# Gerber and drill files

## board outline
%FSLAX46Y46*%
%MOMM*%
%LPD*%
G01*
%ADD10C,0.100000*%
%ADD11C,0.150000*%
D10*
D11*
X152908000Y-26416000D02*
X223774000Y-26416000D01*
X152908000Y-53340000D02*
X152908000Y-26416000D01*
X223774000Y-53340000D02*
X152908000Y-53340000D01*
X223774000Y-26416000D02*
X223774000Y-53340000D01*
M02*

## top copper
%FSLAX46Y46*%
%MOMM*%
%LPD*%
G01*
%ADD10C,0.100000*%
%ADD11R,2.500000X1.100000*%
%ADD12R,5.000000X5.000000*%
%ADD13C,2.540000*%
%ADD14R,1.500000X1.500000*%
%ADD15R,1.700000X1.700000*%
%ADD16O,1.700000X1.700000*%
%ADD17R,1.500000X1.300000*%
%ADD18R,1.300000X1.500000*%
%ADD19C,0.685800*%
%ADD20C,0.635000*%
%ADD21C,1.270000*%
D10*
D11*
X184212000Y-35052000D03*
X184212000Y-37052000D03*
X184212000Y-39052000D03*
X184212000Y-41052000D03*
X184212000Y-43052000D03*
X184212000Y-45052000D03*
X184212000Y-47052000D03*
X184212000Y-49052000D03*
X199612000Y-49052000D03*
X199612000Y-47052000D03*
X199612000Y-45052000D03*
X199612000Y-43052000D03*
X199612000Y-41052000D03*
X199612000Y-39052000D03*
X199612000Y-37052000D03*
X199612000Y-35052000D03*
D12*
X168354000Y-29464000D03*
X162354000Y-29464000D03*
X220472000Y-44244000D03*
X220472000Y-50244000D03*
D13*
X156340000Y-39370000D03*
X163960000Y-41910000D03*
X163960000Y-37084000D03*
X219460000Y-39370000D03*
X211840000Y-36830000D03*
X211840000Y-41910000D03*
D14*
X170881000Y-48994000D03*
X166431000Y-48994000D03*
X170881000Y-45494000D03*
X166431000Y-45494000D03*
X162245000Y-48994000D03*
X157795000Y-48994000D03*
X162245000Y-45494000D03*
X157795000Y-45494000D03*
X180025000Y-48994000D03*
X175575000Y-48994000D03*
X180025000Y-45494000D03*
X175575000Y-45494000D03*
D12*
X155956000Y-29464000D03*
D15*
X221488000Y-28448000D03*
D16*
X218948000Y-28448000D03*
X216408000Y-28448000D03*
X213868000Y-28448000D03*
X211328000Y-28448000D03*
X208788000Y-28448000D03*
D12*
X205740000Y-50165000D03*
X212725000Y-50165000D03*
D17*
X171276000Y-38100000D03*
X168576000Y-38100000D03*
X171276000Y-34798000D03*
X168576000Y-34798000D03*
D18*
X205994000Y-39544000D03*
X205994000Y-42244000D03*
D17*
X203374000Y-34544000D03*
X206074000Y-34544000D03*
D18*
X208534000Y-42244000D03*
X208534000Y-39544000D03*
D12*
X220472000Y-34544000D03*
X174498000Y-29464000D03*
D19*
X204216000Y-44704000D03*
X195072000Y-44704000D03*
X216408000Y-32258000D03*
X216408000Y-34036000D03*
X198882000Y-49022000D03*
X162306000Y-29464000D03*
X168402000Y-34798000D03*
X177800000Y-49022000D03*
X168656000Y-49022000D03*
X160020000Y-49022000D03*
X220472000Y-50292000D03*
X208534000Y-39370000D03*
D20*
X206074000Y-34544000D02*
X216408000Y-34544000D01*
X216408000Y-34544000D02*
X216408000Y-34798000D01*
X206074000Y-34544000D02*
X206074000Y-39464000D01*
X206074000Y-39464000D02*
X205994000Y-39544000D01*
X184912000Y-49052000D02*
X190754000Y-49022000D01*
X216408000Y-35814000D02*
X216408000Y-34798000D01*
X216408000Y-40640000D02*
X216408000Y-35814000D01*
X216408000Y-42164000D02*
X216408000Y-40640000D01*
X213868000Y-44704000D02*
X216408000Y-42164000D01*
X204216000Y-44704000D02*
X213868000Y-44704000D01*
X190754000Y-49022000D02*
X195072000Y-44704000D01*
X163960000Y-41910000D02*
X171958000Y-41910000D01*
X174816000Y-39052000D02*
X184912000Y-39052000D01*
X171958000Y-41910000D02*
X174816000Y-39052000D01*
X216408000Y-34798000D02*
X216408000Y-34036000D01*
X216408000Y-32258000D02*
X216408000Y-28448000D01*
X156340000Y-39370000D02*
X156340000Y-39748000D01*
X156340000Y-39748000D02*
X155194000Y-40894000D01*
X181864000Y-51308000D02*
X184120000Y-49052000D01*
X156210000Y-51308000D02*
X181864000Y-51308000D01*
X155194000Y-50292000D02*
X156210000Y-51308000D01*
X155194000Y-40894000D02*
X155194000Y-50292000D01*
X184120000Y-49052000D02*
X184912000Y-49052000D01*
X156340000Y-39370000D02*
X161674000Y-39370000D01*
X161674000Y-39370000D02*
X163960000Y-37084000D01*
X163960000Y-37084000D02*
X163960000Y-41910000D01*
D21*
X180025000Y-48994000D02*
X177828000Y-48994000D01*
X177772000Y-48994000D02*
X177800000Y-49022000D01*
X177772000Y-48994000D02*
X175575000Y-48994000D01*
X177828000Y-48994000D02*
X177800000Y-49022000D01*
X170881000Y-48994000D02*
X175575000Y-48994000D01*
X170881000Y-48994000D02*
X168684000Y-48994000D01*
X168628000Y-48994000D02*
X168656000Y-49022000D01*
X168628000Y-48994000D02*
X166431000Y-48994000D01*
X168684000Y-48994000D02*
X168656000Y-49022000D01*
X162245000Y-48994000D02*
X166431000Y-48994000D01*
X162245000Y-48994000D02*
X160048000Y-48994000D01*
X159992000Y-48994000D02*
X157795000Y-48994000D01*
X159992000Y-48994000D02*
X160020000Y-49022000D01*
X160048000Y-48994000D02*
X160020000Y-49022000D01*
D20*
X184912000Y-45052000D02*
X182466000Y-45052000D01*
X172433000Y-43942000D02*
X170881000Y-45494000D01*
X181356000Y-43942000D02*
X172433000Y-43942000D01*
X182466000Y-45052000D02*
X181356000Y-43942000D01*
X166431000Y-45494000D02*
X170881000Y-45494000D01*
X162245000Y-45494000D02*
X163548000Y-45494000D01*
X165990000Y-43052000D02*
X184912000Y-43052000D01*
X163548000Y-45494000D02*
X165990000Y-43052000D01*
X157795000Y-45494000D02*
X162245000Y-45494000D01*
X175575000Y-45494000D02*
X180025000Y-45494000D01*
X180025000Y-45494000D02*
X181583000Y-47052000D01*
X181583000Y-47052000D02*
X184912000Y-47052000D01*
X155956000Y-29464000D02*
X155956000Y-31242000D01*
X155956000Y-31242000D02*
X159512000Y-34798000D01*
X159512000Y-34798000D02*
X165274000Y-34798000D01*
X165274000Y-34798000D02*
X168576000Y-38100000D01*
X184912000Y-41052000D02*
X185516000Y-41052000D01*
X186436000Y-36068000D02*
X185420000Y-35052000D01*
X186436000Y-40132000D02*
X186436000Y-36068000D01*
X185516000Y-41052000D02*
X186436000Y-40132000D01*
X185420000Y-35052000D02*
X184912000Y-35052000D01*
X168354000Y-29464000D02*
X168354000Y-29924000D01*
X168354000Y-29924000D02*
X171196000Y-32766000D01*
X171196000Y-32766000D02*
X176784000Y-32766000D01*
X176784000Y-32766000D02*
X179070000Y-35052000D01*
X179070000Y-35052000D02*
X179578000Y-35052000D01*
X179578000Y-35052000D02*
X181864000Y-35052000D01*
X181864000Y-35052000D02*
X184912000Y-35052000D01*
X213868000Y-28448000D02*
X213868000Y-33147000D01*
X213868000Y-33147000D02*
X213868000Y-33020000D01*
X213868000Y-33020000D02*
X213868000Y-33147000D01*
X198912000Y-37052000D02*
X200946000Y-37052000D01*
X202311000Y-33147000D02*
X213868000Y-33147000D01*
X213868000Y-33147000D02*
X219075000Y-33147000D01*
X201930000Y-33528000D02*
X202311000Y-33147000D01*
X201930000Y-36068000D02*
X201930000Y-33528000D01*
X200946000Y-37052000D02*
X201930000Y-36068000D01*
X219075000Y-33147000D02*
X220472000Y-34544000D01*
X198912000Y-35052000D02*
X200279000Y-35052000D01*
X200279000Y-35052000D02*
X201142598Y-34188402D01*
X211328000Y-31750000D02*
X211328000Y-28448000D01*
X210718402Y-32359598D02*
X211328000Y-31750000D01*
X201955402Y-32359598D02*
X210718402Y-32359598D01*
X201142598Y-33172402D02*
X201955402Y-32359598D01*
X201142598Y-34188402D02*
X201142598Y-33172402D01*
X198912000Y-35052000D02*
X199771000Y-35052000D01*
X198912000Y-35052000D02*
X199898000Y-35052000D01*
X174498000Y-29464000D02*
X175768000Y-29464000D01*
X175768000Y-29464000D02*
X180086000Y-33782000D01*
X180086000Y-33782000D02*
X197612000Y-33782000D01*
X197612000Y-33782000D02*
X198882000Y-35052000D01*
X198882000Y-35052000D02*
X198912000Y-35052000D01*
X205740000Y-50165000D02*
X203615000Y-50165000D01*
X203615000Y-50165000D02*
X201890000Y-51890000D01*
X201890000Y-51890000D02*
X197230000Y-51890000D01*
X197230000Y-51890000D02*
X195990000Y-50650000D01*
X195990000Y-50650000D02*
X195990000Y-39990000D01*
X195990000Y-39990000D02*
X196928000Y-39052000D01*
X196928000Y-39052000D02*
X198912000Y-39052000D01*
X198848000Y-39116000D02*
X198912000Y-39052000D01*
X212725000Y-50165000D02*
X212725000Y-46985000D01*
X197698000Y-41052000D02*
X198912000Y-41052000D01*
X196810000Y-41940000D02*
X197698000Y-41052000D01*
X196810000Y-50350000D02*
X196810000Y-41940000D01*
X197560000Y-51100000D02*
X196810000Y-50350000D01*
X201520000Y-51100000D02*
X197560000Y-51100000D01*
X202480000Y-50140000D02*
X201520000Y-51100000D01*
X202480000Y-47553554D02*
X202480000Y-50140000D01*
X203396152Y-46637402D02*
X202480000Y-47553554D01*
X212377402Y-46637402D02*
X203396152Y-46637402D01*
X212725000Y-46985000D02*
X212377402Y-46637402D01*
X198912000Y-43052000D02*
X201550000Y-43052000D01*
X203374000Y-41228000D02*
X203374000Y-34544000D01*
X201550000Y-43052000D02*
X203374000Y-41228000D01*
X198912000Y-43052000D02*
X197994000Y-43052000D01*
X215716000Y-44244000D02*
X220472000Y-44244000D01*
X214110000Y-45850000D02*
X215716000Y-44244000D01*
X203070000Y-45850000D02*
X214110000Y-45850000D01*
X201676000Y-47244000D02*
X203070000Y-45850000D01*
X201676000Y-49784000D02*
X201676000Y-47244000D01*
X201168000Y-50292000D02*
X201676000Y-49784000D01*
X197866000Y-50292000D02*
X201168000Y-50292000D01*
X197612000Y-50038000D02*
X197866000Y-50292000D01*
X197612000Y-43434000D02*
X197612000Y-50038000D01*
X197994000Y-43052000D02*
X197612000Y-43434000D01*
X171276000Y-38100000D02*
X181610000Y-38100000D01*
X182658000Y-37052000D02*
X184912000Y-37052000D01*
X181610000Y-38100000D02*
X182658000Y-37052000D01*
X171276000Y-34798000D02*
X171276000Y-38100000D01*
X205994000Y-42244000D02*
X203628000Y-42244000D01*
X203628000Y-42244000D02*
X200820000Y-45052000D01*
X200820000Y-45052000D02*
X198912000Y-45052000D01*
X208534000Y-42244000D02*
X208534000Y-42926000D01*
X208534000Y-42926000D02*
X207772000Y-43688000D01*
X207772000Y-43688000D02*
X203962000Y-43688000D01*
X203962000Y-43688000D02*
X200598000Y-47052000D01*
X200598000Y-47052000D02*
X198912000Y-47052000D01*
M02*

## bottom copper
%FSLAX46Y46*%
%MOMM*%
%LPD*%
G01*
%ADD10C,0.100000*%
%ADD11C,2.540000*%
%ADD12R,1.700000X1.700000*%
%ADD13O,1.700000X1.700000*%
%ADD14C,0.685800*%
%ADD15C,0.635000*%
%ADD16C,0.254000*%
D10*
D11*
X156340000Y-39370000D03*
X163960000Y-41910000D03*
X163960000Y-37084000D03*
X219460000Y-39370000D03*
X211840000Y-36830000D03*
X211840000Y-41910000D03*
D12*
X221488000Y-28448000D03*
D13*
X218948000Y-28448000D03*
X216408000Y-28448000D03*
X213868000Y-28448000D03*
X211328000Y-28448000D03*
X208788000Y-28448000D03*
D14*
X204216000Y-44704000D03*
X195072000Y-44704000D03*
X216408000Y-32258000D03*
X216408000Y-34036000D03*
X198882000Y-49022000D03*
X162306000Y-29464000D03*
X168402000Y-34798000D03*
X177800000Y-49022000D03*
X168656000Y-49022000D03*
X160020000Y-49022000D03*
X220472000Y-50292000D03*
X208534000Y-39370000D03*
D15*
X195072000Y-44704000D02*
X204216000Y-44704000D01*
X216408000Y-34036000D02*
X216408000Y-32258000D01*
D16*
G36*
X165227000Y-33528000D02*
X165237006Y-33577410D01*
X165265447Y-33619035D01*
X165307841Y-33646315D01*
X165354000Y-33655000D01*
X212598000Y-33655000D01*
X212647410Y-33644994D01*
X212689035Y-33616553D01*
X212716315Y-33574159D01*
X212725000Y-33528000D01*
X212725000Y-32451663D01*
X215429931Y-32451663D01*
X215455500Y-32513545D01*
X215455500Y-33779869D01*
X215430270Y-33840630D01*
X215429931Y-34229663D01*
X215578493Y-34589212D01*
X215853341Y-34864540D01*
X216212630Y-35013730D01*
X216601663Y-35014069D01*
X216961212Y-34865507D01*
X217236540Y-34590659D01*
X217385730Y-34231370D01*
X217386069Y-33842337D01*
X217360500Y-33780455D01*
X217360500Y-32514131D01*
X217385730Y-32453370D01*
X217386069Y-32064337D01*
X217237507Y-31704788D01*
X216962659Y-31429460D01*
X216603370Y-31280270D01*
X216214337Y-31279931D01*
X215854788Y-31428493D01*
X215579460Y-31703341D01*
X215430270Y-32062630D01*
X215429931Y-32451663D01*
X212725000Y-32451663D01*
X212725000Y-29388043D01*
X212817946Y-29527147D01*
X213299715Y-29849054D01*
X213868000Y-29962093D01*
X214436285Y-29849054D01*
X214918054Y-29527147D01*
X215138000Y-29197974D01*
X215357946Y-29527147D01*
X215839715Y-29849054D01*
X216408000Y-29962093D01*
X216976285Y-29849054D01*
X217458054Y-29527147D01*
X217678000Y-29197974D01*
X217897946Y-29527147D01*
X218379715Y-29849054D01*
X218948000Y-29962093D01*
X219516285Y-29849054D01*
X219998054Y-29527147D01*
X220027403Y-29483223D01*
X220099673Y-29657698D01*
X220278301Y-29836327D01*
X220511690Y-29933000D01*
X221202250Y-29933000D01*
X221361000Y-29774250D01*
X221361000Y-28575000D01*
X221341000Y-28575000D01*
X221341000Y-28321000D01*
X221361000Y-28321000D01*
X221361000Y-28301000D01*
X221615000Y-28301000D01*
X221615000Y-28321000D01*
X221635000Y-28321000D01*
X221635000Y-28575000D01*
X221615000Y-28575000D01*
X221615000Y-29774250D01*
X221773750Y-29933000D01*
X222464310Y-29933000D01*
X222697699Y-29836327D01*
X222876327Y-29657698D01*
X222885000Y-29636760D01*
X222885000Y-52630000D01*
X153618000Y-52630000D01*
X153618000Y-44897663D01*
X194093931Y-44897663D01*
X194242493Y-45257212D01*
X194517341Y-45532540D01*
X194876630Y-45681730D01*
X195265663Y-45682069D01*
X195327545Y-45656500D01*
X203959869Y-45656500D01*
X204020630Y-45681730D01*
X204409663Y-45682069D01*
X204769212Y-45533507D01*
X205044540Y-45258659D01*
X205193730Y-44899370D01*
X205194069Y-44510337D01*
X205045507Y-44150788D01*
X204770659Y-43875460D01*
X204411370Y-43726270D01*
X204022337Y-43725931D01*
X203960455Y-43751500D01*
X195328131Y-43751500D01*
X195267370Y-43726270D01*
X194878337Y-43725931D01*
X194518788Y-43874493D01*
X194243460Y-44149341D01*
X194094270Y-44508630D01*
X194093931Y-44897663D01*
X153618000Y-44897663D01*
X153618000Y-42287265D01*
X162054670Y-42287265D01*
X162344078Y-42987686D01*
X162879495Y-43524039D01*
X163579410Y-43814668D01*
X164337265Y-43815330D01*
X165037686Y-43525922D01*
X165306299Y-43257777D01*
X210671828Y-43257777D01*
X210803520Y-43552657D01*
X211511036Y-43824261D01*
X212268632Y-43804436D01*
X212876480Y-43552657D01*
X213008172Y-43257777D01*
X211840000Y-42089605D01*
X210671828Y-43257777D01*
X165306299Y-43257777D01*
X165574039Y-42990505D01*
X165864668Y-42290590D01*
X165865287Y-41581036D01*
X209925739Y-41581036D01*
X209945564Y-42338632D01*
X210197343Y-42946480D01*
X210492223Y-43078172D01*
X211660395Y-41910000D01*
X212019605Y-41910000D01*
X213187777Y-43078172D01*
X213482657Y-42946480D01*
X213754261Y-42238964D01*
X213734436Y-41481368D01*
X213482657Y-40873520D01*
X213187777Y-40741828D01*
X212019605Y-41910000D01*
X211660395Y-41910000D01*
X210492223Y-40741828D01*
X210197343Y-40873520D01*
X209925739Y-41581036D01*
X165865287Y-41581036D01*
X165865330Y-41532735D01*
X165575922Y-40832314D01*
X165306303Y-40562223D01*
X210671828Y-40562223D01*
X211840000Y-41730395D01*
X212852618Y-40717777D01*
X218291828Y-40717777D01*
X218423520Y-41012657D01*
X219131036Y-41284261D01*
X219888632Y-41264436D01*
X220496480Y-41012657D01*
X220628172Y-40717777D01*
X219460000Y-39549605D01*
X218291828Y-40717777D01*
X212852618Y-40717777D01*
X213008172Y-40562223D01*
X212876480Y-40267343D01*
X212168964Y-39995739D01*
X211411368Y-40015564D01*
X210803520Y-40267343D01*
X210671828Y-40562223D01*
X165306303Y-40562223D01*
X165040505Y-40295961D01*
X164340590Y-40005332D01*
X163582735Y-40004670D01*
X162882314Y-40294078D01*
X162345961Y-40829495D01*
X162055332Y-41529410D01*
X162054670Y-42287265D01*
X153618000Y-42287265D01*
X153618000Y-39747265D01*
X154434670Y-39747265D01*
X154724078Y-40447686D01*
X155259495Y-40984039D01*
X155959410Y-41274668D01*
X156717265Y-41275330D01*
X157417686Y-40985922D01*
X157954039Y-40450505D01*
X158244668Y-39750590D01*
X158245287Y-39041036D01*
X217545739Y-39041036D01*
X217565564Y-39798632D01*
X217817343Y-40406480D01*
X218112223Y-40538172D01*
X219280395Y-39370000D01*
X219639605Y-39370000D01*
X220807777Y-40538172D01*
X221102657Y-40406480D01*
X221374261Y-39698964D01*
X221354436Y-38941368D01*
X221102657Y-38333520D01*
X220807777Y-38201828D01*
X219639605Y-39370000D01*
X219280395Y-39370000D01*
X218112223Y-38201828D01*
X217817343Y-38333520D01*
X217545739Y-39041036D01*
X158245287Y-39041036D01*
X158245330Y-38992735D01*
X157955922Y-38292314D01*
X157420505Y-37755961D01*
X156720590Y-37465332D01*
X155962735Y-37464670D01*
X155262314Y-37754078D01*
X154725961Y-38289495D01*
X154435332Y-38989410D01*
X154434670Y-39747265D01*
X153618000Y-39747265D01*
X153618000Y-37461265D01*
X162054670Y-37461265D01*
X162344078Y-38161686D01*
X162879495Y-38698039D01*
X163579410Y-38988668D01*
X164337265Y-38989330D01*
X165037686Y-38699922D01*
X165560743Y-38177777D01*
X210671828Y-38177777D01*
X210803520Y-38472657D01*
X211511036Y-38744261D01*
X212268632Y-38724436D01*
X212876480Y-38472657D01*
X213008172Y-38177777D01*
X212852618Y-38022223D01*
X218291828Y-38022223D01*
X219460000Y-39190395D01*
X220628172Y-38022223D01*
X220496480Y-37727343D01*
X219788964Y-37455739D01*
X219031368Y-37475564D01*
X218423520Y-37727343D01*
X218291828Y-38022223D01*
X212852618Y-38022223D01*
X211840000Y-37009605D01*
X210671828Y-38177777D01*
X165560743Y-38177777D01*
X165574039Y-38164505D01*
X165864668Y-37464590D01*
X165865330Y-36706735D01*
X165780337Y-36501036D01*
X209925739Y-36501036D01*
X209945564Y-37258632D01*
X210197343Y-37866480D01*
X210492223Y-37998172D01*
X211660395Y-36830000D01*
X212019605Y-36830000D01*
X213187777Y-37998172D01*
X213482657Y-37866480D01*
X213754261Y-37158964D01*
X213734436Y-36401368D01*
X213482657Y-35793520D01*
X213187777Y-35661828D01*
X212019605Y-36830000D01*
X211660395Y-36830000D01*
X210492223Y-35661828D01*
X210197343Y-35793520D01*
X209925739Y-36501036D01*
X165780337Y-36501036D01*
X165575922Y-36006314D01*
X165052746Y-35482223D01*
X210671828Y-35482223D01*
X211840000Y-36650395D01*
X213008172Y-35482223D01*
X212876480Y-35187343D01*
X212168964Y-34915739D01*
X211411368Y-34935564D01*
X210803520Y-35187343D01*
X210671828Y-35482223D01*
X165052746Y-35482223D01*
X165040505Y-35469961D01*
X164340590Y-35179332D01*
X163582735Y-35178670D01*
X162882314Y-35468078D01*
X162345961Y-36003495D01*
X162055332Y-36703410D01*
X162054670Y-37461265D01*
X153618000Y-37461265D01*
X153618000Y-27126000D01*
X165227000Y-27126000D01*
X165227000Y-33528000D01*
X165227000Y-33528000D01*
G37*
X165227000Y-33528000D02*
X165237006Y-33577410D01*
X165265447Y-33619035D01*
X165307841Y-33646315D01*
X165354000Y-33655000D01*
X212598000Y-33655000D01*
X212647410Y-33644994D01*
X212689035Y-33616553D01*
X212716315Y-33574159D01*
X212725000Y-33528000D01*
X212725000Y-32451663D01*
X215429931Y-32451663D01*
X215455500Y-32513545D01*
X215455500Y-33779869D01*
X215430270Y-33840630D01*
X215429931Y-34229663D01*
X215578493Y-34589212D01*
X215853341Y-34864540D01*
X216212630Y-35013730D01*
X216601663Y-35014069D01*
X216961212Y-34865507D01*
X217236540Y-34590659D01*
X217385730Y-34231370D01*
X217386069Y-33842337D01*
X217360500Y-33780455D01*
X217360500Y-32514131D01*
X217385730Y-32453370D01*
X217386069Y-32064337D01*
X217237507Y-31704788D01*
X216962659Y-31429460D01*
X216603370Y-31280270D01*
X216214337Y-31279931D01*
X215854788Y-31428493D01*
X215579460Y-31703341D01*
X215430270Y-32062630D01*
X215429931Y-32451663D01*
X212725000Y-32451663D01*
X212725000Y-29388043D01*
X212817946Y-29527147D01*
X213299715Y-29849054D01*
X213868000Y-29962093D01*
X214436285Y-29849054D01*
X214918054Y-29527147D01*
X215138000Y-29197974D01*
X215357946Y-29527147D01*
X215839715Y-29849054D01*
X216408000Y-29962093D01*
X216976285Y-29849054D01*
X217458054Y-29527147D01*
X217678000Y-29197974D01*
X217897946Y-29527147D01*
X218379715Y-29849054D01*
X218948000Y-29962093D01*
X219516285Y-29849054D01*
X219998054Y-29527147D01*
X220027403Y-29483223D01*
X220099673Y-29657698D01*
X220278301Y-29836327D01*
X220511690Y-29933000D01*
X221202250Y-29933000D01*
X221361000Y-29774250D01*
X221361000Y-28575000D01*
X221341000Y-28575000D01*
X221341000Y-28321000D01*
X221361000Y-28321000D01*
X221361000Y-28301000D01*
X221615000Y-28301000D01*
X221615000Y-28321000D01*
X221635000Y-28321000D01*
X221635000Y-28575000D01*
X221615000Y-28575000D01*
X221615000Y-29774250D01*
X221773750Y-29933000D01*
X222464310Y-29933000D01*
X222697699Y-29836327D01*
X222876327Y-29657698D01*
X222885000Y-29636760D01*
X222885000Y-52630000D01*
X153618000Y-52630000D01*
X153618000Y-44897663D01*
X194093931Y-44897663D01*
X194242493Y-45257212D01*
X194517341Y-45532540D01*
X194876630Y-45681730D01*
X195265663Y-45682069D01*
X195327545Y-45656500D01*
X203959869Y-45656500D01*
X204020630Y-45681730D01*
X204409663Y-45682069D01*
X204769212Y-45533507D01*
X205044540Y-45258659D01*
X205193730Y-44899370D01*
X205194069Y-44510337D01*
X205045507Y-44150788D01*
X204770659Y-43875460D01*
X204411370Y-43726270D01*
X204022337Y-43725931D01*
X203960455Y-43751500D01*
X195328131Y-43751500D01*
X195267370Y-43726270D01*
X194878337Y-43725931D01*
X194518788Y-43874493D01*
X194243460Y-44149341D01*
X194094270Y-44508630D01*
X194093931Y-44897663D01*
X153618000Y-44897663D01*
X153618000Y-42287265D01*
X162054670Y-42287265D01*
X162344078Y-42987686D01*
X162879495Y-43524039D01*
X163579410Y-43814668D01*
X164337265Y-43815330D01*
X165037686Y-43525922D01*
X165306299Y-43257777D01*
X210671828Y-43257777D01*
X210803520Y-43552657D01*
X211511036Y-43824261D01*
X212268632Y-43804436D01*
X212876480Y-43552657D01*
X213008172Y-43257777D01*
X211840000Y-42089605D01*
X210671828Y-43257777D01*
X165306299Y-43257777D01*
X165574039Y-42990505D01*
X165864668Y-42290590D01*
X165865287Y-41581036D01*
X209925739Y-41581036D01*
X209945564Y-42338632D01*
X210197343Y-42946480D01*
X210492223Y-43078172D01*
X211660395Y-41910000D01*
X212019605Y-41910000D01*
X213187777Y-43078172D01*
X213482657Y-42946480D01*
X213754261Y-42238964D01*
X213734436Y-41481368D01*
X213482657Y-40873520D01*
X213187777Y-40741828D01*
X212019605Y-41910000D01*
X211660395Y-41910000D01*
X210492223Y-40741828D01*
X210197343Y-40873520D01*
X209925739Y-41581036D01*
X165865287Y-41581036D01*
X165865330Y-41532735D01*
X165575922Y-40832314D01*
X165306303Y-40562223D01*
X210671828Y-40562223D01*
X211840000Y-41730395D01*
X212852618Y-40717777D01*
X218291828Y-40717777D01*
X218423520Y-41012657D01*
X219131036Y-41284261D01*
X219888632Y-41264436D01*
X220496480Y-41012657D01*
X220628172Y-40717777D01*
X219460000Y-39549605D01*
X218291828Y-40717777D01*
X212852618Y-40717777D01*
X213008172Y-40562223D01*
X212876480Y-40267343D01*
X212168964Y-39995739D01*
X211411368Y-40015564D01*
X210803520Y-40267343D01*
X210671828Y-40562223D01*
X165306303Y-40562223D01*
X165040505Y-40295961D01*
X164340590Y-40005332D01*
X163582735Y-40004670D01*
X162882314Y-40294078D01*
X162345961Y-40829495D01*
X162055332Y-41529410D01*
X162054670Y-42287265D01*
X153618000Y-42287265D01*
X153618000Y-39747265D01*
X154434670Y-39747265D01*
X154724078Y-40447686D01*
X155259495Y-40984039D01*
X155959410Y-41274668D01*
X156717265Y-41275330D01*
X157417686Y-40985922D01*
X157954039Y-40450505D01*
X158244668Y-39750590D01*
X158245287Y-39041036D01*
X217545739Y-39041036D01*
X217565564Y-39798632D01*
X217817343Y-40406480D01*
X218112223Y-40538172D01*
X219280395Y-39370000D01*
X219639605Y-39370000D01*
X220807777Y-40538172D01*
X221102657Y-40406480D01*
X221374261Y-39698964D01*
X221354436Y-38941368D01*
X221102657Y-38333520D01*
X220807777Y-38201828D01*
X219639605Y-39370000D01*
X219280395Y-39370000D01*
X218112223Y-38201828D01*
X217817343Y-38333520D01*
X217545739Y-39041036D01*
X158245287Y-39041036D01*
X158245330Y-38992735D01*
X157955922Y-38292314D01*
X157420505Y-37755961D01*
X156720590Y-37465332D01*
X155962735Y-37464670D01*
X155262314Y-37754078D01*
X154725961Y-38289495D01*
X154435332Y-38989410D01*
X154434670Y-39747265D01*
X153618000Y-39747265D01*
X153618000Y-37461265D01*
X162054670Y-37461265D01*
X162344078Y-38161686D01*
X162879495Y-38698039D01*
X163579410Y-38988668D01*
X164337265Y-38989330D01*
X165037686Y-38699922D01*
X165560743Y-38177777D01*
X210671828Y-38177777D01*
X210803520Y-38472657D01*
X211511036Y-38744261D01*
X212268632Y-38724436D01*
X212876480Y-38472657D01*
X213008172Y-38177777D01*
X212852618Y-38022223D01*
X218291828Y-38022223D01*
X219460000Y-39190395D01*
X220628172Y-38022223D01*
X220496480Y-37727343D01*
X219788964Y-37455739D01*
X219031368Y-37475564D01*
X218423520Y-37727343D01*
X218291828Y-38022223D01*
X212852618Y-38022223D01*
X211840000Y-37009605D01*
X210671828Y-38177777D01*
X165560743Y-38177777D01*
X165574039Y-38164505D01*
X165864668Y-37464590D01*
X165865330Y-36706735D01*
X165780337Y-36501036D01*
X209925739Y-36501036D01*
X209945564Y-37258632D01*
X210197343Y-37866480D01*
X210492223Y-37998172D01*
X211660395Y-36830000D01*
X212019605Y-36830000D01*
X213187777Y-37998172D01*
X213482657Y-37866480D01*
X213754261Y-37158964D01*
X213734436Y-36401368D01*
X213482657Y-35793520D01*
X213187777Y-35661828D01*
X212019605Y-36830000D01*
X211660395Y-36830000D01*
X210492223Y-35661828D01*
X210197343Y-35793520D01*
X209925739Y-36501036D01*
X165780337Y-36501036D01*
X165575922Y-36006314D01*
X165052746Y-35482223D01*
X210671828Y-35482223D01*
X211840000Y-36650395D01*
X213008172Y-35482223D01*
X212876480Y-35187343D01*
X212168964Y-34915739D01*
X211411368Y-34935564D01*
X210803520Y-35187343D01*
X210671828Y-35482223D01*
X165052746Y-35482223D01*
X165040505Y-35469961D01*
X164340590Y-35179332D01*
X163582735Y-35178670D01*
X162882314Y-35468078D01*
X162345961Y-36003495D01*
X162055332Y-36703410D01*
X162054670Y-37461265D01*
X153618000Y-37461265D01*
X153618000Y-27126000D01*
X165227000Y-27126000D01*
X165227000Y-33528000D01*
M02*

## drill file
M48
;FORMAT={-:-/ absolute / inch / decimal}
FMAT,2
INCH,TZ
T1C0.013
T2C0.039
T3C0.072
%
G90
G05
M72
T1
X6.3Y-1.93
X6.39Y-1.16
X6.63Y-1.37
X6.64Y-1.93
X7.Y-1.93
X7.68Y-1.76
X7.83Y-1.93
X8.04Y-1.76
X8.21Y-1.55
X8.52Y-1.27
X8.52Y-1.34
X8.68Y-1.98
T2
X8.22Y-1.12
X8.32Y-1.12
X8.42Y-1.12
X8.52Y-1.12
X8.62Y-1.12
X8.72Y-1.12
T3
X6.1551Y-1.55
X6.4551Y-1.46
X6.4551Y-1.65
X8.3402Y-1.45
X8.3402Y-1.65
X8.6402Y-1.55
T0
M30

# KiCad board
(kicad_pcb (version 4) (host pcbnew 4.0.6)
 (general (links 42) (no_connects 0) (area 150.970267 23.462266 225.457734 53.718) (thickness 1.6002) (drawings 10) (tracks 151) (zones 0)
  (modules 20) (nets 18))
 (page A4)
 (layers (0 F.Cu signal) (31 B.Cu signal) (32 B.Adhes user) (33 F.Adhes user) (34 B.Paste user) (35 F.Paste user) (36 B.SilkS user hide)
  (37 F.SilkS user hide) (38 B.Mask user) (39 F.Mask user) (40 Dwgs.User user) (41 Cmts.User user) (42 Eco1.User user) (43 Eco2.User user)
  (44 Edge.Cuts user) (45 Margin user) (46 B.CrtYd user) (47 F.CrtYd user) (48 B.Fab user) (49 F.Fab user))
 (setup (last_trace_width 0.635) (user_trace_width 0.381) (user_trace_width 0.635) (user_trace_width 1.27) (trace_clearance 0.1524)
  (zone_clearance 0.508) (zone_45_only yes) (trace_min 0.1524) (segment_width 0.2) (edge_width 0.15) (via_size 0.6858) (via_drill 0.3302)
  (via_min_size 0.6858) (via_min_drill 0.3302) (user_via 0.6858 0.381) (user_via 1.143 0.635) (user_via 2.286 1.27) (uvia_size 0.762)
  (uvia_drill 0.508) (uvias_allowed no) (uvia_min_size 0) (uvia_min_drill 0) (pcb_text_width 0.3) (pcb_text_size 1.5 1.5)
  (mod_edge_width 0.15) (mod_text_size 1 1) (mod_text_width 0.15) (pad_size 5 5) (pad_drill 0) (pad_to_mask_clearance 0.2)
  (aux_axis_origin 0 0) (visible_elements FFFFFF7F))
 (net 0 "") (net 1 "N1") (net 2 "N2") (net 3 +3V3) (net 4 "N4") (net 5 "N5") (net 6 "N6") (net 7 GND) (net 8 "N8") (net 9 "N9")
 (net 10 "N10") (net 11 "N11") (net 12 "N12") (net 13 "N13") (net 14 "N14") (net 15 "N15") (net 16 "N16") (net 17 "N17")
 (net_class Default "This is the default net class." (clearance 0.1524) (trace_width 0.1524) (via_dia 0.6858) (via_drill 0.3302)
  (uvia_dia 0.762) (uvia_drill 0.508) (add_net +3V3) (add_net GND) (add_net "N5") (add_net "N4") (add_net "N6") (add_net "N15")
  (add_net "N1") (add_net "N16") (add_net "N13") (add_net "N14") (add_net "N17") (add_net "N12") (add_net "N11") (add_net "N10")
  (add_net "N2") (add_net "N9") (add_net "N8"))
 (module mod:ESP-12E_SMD (layer F.Cu) (at 184.912 35.052)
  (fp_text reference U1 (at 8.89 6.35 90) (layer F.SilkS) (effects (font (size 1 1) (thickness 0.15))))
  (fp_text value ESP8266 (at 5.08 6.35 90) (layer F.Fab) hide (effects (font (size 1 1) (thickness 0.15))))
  (pad 1 smd rect (at 0 0) (size 2.5 1.1) (drill (offset -0.7 0)) (layers F.Cu F.Paste F.Mask) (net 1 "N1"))
  (pad 2 smd rect (at 0 2) (size 2.5 1.1) (drill (offset -0.7 0)) (layers F.Cu F.Paste F.Mask) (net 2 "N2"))
  (pad 3 smd rect (at 0 4) (size 2.5 1.1) (drill (offset -0.7 0)) (layers F.Cu F.Paste F.Mask) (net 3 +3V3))
  (pad 4 smd rect (at 0 6) (size 2.5 1.1) (drill (offset -0.7 0)) (layers F.Cu F.Paste F.Mask) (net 1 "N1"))
  (pad 5 smd rect (at 0 8) (size 2.5 1.1) (drill (offset -0.7 0)) (layers F.Cu F.Paste F.Mask) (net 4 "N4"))
  (pad 6 smd rect (at 0 10) (size 2.5 1.1) (drill (offset -0.7 0)) (layers F.Cu F.Paste F.Mask) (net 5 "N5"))
  (pad 7 smd rect (at 0 12) (size 2.5 1.1) (drill (offset -0.7 0)) (layers F.Cu F.Paste F.Mask) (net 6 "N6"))
  (pad 8 smd rect (at 0 14) (size 2.5 1.1) (drill (offset -0.7 0)) (layers F.Cu F.Paste F.Mask) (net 3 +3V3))
  (pad 9 smd rect (at 14 14) (size 2.5 1.1) (drill (offset 0.7 0)) (layers F.Cu F.Paste F.Mask) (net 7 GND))
  (pad 10 smd rect (at 14 12) (size 2.5 1.1) (drill (offset 0.7 0)) (layers F.Cu F.Paste F.Mask) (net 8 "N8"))
  (pad 11 smd rect (at 14 10) (size 2.5 1.1) (drill (offset 0.7 0)) (layers F.Cu F.Paste F.Mask) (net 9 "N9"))
  (pad 12 smd rect (at 14 8) (size 2.5 1.1) (drill (offset 0.7 0)) (layers F.Cu F.Paste F.Mask) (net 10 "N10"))
  (pad 13 smd rect (at 14 6) (size 2.5 1.1) (drill (offset 0.7 0)) (layers F.Cu F.Paste F.Mask) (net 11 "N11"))
  (pad 14 smd rect (at 14 4) (size 2.5 1.1) (drill (offset 0.7 0)) (layers F.Cu F.Paste F.Mask) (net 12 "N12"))
  (pad 15 smd rect (at 14 2) (size 2.5 1.1) (drill (offset 0.7 0)) (layers F.Cu F.Paste F.Mask) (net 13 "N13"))
  (pad 16 smd rect (at 14 0) (size 2.5 1.1) (drill (offset 0.7 0)) (layers F.Cu F.Paste F.Mask) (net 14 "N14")))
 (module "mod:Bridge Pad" (layer F.Cu) (at 165.354 29.464)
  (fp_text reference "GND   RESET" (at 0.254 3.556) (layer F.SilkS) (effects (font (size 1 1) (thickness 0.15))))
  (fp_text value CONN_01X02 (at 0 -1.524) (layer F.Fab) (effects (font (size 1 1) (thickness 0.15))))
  (pad 1 smd rect (at 3 0) (size 5 5) (layers F.Cu F.Mask) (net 1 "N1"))
  (pad 2 smd rect (at -3 0) (size 5 5) (layers F.Cu F.Mask) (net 7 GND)))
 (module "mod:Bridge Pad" (layer F.Cu) (at 220.472 47.244 90)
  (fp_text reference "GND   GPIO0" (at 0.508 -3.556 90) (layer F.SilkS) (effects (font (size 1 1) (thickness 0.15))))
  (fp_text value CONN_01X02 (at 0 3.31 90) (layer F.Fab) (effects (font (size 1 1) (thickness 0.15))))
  (pad 1 smd rect (at 3 0 90) (size 5 5) (layers F.Cu F.Mask) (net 10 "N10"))
  (pad 2 smd rect (at -3 0 90) (size 5 5) (layers F.Cu F.Mask) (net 7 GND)))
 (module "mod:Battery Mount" (layer F.Cu) (at 187.96 39.37 90)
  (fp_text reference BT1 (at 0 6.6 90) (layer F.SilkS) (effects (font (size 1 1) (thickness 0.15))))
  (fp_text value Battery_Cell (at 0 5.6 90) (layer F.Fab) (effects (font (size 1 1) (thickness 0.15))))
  (pad 1 thru_hole circle (at 0 -31.62 90) (size 2.54 2.54) (drill 1.8288) (layers *.Cu *.Mask) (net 3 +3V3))
  (pad 1 thru_hole circle (at -2.54 -24 90) (size 2.54 2.54) (drill 1.8288) (layers *.Cu *.Mask) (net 3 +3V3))
  (pad 1 thru_hole circle (at 2.286 -24 90) (size 2.54 2.54) (drill 1.8288) (layers *.Cu *.Mask) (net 3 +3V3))
  (pad 2 thru_hole circle (at 0 31.5 90) (size 2.54 2.54) (drill 1.8288) (layers *.Cu *.Mask) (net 7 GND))
  (pad 2 thru_hole circle (at 2.54 23.88 90) (size 2.54 2.54) (drill 1.8288) (layers *.Cu *.Mask) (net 7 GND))
  (pad 2 thru_hole circle (at -2.54 23.88 90) (size 2.54 2.54) (drill 1.8288) (layers *.Cu *.Mask) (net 7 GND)))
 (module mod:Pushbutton (layer F.Cu) (at 168.656 47.244 180)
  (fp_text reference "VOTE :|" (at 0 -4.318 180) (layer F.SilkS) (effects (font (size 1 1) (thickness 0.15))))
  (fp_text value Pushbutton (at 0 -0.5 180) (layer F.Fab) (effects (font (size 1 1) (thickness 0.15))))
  (pad 1 smd rect (at -2.225 -1.75 180) (size 1.5 1.5) (layers F.Cu F.Paste F.Mask) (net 7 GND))
  (pad 1 smd rect (at 2.225 -1.75 180) (size 1.5 1.5) (layers F.Cu F.Paste F.Mask) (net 7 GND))
  (pad 2 smd rect (at -2.225 1.75 180) (size 1.5 1.5) (layers F.Cu F.Paste F.Mask) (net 5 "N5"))
  (pad 2 smd rect (at 2.225 1.75 180) (size 1.5 1.5) (layers F.Cu F.Paste F.Mask) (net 5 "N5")))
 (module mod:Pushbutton (layer F.Cu) (at 160.02 47.244 180)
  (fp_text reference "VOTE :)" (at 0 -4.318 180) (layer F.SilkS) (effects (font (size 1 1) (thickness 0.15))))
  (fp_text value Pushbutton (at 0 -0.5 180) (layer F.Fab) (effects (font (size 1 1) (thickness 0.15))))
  (pad 1 smd rect (at -2.225 -1.75 180) (size 1.5 1.5) (layers F.Cu F.Paste F.Mask) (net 7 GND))
  (pad 1 smd rect (at 2.225 -1.75 180) (size 1.5 1.5) (layers F.Cu F.Paste F.Mask) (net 7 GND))
  (pad 2 smd rect (at -2.225 1.75 180) (size 1.5 1.5) (layers F.Cu F.Paste F.Mask) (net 4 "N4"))
  (pad 2 smd rect (at 2.225 1.75 180) (size 1.5 1.5) (layers F.Cu F.Paste F.Mask) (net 4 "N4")))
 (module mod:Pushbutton (layer F.Cu) (at 177.8 47.244 180)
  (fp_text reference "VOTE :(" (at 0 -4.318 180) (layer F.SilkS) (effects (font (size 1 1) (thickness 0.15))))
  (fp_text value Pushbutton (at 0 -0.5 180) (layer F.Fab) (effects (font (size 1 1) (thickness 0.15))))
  (pad 1 smd rect (at -2.225 -1.75 180) (size 1.5 1.5) (layers F.Cu F.Paste F.Mask) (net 7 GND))
  (pad 1 smd rect (at 2.225 -1.75 180) (size 1.5 1.5) (layers F.Cu F.Paste F.Mask) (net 7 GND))
  (pad 2 smd rect (at -2.225 1.75 180) (size 1.5 1.5) (layers F.Cu F.Paste F.Mask) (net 6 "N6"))
  (pad 2 smd rect (at 2.225 1.75 180) (size 1.5 1.5) (layers F.Cu F.Paste F.Mask) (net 6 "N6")))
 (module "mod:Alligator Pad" (layer F.Cu) (at 155.956 29.464)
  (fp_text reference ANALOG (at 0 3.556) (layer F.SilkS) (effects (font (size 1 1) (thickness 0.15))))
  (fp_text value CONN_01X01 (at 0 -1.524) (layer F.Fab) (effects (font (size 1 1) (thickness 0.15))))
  (pad 1 smd rect (at 0 0) (size 5 5) (layers F.Cu F.Mask) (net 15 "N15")))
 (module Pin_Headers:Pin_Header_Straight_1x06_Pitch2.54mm (layer F.Cu) (at 221.488 28.448 270)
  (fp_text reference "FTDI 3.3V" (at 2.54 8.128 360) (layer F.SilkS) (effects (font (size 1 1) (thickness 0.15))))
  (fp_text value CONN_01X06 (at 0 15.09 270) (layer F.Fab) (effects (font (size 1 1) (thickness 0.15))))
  (pad 1 thru_hole rect (at 0 0 270) (size 1.7 1.7) (drill 1) (layers *.Cu *.Mask) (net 7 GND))
  (pad 2 thru_hole oval (at 0 2.54 270) (size 1.7 1.7) (drill 1) (layers *.Cu *.Mask) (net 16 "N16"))
  (pad 3 thru_hole oval (at 0 5.08 270) (size 1.7 1.7) (drill 1) (layers *.Cu *.Mask) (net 3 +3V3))
  (pad 4 thru_hole oval (at 0 7.62 270) (size 1.7 1.7) (drill 1) (layers *.Cu *.Mask) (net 13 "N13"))
  (pad 5 thru_hole oval (at 0 10.16 270) (size 1.7 1.7) (drill 1) (layers *.Cu *.Mask) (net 14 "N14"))
  (pad 6 thru_hole oval (at 0 12.7 270) (size 1.7 1.7) (drill 1) (layers *.Cu *.Mask) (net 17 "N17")))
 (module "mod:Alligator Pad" (layer F.Cu) (at 205.74 50.165)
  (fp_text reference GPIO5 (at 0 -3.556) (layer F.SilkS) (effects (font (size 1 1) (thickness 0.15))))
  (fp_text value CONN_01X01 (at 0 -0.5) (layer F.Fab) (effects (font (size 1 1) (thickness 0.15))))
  (pad 1 smd rect (at 0 0) (size 5 5) (layers F.Cu F.Mask) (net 12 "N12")))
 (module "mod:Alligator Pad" (layer F.Cu) (at 212.725 50.165)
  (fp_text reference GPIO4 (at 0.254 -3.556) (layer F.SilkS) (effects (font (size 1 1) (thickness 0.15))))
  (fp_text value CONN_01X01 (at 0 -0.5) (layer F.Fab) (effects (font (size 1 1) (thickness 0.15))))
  (pad 1 smd rect (at 0 0) (size 5 5) (layers F.Cu F.Mask) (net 11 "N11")))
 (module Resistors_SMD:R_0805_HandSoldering (layer F.Cu) (at 169.926 38.1 180)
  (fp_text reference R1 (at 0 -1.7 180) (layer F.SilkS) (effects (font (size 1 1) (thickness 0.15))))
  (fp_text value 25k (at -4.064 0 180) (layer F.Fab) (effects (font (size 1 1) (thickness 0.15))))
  (pad 1 smd rect (at -1.35 0 180) (size 1.5 1.3) (layers F.Cu F.Paste F.Mask) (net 2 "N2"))
  (pad 2 smd rect (at 1.35 0 180) (size 1.5 1.3) (layers F.Cu F.Paste F.Mask) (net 15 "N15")))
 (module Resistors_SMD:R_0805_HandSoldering (layer F.Cu) (at 169.926 34.798 180)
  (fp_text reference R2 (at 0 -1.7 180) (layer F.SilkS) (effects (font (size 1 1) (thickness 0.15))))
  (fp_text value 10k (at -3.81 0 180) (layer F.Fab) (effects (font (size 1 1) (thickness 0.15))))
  (pad 1 smd rect (at -1.35 0 180) (size 1.5 1.3) (layers F.Cu F.Paste F.Mask) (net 2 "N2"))
  (pad 2 smd rect (at 1.35 0 180) (size 1.5 1.3) (layers F.Cu F.Paste F.Mask) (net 7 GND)))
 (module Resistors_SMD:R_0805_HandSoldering (layer F.Cu) (at 205.994 40.894 270)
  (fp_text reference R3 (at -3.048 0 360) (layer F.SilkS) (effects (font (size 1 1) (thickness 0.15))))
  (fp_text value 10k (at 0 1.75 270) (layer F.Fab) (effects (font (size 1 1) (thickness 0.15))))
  (pad 1 smd rect (at -1.35 0 270) (size 1.5 1.3) (layers F.Cu F.Paste F.Mask) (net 3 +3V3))
  (pad 2 smd rect (at 1.35 0 270) (size 1.5 1.3) (layers F.Cu F.Paste F.Mask) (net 9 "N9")))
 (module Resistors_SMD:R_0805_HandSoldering (layer F.Cu) (at 204.724 34.544)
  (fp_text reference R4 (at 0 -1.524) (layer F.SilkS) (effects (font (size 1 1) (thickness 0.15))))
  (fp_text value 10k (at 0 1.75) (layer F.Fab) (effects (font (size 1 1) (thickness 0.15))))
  (pad 1 smd rect (at -1.35 0) (size 1.5 1.3) (layers F.Cu F.Paste F.Mask) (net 10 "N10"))
  (pad 2 smd rect (at 1.35 0) (size 1.5 1.3) (layers F.Cu F.Paste F.Mask) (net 3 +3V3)))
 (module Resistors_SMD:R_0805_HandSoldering (layer F.Cu) (at 208.534 40.894 90)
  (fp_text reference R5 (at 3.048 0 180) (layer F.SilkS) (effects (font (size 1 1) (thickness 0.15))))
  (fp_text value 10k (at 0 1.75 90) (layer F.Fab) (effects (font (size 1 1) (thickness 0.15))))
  (pad 1 smd rect (at -1.35 0 90) (size 1.5 1.3) (layers F.Cu F.Paste F.Mask) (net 8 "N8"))
  (pad 2 smd rect (at 1.35 0 90) (size 1.5 1.3) (layers F.Cu F.Paste F.Mask) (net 7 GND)))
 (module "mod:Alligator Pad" (layer F.Cu) (at 220.472 34.544)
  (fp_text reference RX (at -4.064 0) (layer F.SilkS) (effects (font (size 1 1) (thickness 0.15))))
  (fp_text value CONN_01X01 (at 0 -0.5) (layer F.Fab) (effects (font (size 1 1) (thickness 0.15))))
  (pad 1 smd rect (at 0 0) (size 5 5) (layers F.Cu F.Mask) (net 13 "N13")))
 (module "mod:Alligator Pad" (layer F.Cu) (at 174.498 29.464)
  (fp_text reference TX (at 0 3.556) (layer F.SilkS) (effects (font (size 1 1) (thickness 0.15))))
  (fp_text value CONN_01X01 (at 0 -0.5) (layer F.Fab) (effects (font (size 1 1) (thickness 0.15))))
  (pad 1 smd rect (at 0 0) (size 5 5) (layers F.Cu F.Mask) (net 14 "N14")))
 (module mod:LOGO (layer F.Cu) (at 177.292 38.1)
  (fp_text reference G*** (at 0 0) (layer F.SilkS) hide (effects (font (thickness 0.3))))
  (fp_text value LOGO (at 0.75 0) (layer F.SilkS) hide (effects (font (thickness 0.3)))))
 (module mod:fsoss (layer B.Cu) (at 159.258 47.244)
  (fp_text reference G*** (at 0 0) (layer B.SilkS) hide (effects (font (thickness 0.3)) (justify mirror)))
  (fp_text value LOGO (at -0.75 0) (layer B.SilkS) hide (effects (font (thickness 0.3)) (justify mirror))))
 (gr_line (start 152.908 26.416) (end 223.774 26.416) (angle 90) (layer Edge.Cuts) (width 0.15))
 (gr_line (start 152.908 53.34) (end 152.908 26.416) (angle 90) (layer Edge.Cuts) (width 0.15))
 (gr_line (start 223.774 53.34) (end 152.908 53.34) (angle 90) (layer Edge.Cuts) (width 0.15))
 (gr_line (start 223.774 26.416) (end 223.774 53.34) (angle 90) (layer Edge.Cuts) (width 0.15))
 (segment (start 206.074 34.544) (end 216.408 34.544) (width 0.635) (layer F.Cu) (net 3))
 (segment (start 216.408 34.544) (end 216.408 34.798) (width 0.635) (layer F.Cu) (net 3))
 (segment (start 206.074 34.544) (end 206.074 39.464) (width 0.635) (layer F.Cu) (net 3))
 (segment (start 206.074 39.464) (end 205.994 39.544) (width 0.635) (layer F.Cu) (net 3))
 (segment (start 184.912 49.052) (end 190.754 49.022) (width 0.635) (layer F.Cu) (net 3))
 (segment (start 216.408 35.814) (end 216.408 34.798) (width 0.635) (layer F.Cu) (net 3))
 (segment (start 216.408 40.64) (end 216.408 35.814) (width 0.635) (layer F.Cu) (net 3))
 (segment (start 216.408 42.164) (end 216.408 40.64) (width 0.635) (layer F.Cu) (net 3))
 (segment (start 213.868 44.704) (end 216.408 42.164) (width 0.635) (layer F.Cu) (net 3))
 (segment (start 204.216 44.704) (end 213.868 44.704) (width 0.635) (layer F.Cu) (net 3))
 (via (at 204.216 44.704) (size 0.6858) (drill 0.3302) (layers F.Cu B.Cu) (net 3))
 (segment (start 195.072 44.704) (end 204.216 44.704) (width 0.635) (layer B.Cu) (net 3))
 (via (at 195.072 44.704) (size 0.6858) (drill 0.3302) (layers F.Cu B.Cu) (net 3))
 (segment (start 190.754 49.022) (end 195.072 44.704) (width 0.635) (layer F.Cu) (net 3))
 (segment (start 163.96 41.91) (end 171.958 41.91) (width 0.635) (layer F.Cu) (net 3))
 (segment (start 174.816 39.052) (end 184.912 39.052) (width 0.635) (layer F.Cu) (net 3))
 (segment (start 171.958 41.91) (end 174.816 39.052) (width 0.635) (layer F.Cu) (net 3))
 (segment (start 216.408 34.798) (end 216.408 34.036) (width 0.635) (layer F.Cu) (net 3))
 (segment (start 216.408 32.258) (end 216.408 28.448) (width 0.635) (layer F.Cu) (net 3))
 (via (at 216.408 32.258) (size 0.6858) (drill 0.3302) (layers F.Cu B.Cu) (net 3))
 (segment (start 216.408 34.036) (end 216.408 32.258) (width 0.635) (layer B.Cu) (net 3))
 (via (at 216.408 34.036) (size 0.6858) (drill 0.3302) (layers F.Cu B.Cu) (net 3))
 (segment (start 156.34 39.37) (end 156.34 39.748) (width 0.635) (layer F.Cu) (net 3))
 (segment (start 156.34 39.748) (end 155.194 40.894) (width 0.635) (layer F.Cu) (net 3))
 (segment (start 181.864 51.308) (end 184.12 49.052) (width 0.635) (layer F.Cu) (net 3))
 (segment (start 156.21 51.308) (end 181.864 51.308) (width 0.635) (layer F.Cu) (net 3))
 (segment (start 155.194 50.292) (end 156.21 51.308) (width 0.635) (layer F.Cu) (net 3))
 (segment (start 155.194 40.894) (end 155.194 50.292) (width 0.635) (layer F.Cu) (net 3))
 (segment (start 184.12 49.052) (end 184.912 49.052) (width 0.635) (layer F.Cu) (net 3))
 (segment (start 156.34 39.37) (end 161.674 39.37) (width 0.635) (layer F.Cu) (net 3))
 (segment (start 161.674 39.37) (end 163.96 37.084) (width 0.635) (layer F.Cu) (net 3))
 (segment (start 163.96 37.084) (end 163.96 41.91) (width 0.635) (layer F.Cu) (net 3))
 (via (at 198.882 49.022) (size 0.6858) (drill 0.3302) (layers F.Cu B.Cu) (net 7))
 (via (at 162.306 29.464) (size 0.6858) (drill 0.3302) (layers F.Cu B.Cu) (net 7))
 (via (at 168.402 34.798) (size 0.6858) (drill 0.3302) (layers F.Cu B.Cu) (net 7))
 (segment (start 180.025 48.994) (end 177.828 48.994) (width 1.27) (layer F.Cu) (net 7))
 (segment (start 177.772 48.994) (end 177.8 49.022) (width 1.27) (layer F.Cu) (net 7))
 (via (at 177.8 49.022) (size 0.6858) (drill 0.3302) (layers F.Cu B.Cu) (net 7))
 (segment (start 177.772 48.994) (end 175.575 48.994) (width 1.27) (layer F.Cu) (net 7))
 (segment (start 177.828 48.994) (end 177.8 49.022) (width 1.27) (layer F.Cu) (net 7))
 (segment (start 170.881 48.994) (end 175.575 48.994) (width 1.27) (layer F.Cu) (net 7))
 (segment (start 170.881 48.994) (end 168.684 48.994) (width 1.27) (layer F.Cu) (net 7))
 (segment (start 168.628 48.994) (end 168.656 49.022) (width 1.27) (layer F.Cu) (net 7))
 (via (at 168.656 49.022) (size 0.6858) (drill 0.3302) (layers F.Cu B.Cu) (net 7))
 (segment (start 168.628 48.994) (end 166.431 48.994) (width 1.27) (layer F.Cu) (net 7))
 (segment (start 168.684 48.994) (end 168.656 49.022) (width 1.27) (layer F.Cu) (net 7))
 (segment (start 162.245 48.994) (end 166.431 48.994) (width 1.27) (layer F.Cu) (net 7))
 (segment (start 162.245 48.994) (end 160.048 48.994) (width 1.27) (layer F.Cu) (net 7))
 (segment (start 159.992 48.994) (end 157.795 48.994) (width 1.27) (layer F.Cu) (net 7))
 (via (at 160.02 49.022) (size 0.6858) (drill 0.3302) (layers F.Cu B.Cu) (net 7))
 (segment (start 159.992 48.994) (end 160.02 49.022) (width 1.27) (layer F.Cu) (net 7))
 (segment (start 160.048 48.994) (end 160.02 49.022) (width 1.27) (layer F.Cu) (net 7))
 (via (at 220.472 50.292) (size 0.6858) (drill 0.3302) (layers F.Cu B.Cu) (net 7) (status 30))
 (via (at 208.534 39.37) (size 0.6858) (drill 0.3302) (layers F.Cu B.Cu) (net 7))
 (segment (start 184.912 45.052) (end 182.466 45.052) (width 0.635) (layer F.Cu) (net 5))
 (segment (start 172.433 43.942) (end 170.881 45.494) (width 0.635) (layer F.Cu) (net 5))
 (segment (start 181.356 43.942) (end 172.433 43.942) (width 0.635) (layer F.Cu) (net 5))
 (segment (start 182.466 45.052) (end 181.356 43.942) (width 0.635) (layer F.Cu) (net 5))
 (segment (start 166.431 45.494) (end 170.881 45.494) (width 0.635) (layer F.Cu) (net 5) (status 30))
 (segment (start 162.245 45.494) (end 163.548 45.494) (width 0.635) (layer F.Cu) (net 4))
 (segment (start 165.99 43.052) (end 184.912 43.052) (width 0.635) (layer F.Cu) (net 4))
 (segment (start 163.548 45.494) (end 165.99 43.052) (width 0.635) (layer F.Cu) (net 4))
 (segment (start 157.795 45.494) (end 162.245 45.494) (width 0.635) (layer F.Cu) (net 4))
 (segment (start 175.575 45.494) (end 180.025 45.494) (width 0.635) (layer F.Cu) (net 6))
 (segment (start 180.025 45.494) (end 181.583 47.052) (width 0.635) (layer F.Cu) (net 6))
 (segment (start 181.583 47.052) (end 184.912 47.052) (width 0.635) (layer F.Cu) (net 6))
 (segment (start 155.956 29.464) (end 155.956 31.242) (width 0.635) (layer F.Cu) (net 15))
 (segment (start 155.956 31.242) (end 159.512 34.798) (width 0.635) (layer F.Cu) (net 15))
 (segment (start 159.512 34.798) (end 165.274 34.798) (width 0.635) (layer F.Cu) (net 15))
 (segment (start 165.274 34.798) (end 168.576 38.1) (width 0.635) (layer F.Cu) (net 15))
 (segment (start 184.912 41.052) (end 185.516 41.052) (width 0.635) (layer F.Cu) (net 1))
 (segment (start 186.436 36.068) (end 185.42 35.052) (width 0.635) (layer F.Cu) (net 1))
 (segment (start 186.436 40.132) (end 186.436 36.068) (width 0.635) (layer F.Cu) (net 1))
 (segment (start 185.516 41.052) (end 186.436 40.132) (width 0.635) (layer F.Cu) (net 1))
 (segment (start 185.42 35.052) (end 184.912 35.052) (width 0.635) (layer F.Cu) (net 1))
 (segment (start 168.354 29.464) (end 168.354 29.924) (width 0.635) (layer F.Cu) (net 1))
 (segment (start 168.354 29.924) (end 171.196 32.766) (width 0.635) (layer F.Cu) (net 1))
 (segment (start 171.196 32.766) (end 176.784 32.766) (width 0.635) (layer F.Cu) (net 1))
 (segment (start 176.784 32.766) (end 179.07 35.052) (width 0.635) (layer F.Cu) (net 1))
 (segment (start 179.07 35.052) (end 179.578 35.052) (width 0.635) (layer F.Cu) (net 1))
 (segment (start 179.578 35.052) (end 181.864 35.052) (width 0.635) (layer F.Cu) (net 1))
 (segment (start 181.864 35.052) (end 184.912 35.052) (width 0.635) (layer F.Cu) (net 1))
 (segment (start 213.868 28.448) (end 213.868 33.147) (width 0.635) (layer F.Cu) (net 13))
 (segment (start 213.868 33.147) (end 213.868 33.02) (width 0.635) (layer F.Cu) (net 13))
 (segment (start 213.868 33.02) (end 213.868 33.147) (width 0.635) (layer F.Cu) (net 13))
 (segment (start 198.912 37.052) (end 200.946 37.052) (width 0.635) (layer F.Cu) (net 13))
 (segment (start 202.311 33.147) (end 213.868 33.147) (width 0.635) (layer F.Cu) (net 13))
 (segment (start 213.868 33.147) (end 219.075 33.147) (width 0.635) (layer F.Cu) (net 13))
 (segment (start 201.93 33.528) (end 202.311 33.147) (width 0.635) (layer F.Cu) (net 13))
 (segment (start 201.93 36.068) (end 201.93 33.528) (width 0.635) (layer F.Cu) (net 13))
 (segment (start 200.946 37.052) (end 201.93 36.068) (width 0.635) (layer F.Cu) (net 13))
 (segment (start 219.075 33.147) (end 220.472 34.544) (width 0.635) (layer F.Cu) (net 13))
 (segment (start 198.912 35.052) (end 200.279 35.052) (width 0.635) (layer F.Cu) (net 14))
 (segment (start 200.279 35.052) (end 201.142598 34.188402) (width 0.635) (layer F.Cu) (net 14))
 (segment (start 211.328 31.75) (end 211.328 28.448) (width 0.635) (layer F.Cu) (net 14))
 (segment (start 210.718402 32.359598) (end 211.328 31.75) (width 0.635) (layer F.Cu) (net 14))
 (segment (start 201.955402 32.359598) (end 210.718402 32.359598) (width 0.635) (layer F.Cu) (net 14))
 (segment (start 201.142598 33.172402) (end 201.955402 32.359598) (width 0.635) (layer F.Cu) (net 14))
 (segment (start 201.142598 34.188402) (end 201.142598 33.172402) (width 0.635) (layer F.Cu) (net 14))
 (segment (start 198.912 35.052) (end 199.771 35.052) (width 0.635) (layer F.Cu) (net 14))
 (segment (start 198.912 35.052) (end 199.898 35.052) (width 0.635) (layer F.Cu) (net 14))
 (segment (start 174.498 29.464) (end 175.768 29.464) (width 0.635) (layer F.Cu) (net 14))
 (segment (start 175.768 29.464) (end 180.086 33.782) (width 0.635) (layer F.Cu) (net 14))
 (segment (start 180.086 33.782) (end 197.612 33.782) (width 0.635) (layer F.Cu) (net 14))
 (segment (start 197.612 33.782) (end 198.882 35.052) (width 0.635) (layer F.Cu) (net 14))
 (segment (start 198.882 35.052) (end 198.912 35.052) (width 0.635) (layer F.Cu) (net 14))
 (segment (start 205.74 50.165) (end 203.615 50.165) (width 0.635) (layer F.Cu) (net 12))
 (segment (start 203.615 50.165) (end 201.89 51.89) (width 0.635) (layer F.Cu) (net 12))
 (segment (start 201.89 51.89) (end 197.23 51.89) (width 0.635) (layer F.Cu) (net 12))
 (segment (start 197.23 51.89) (end 195.99 50.65) (width 0.635) (layer F.Cu) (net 12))
 (segment (start 195.99 50.65) (end 195.99 39.99) (width 0.635) (layer F.Cu) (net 12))
 (segment (start 195.99 39.99) (end 196.928 39.052) (width 0.635) (layer F.Cu) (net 12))
 (segment (start 196.928 39.052) (end 198.912 39.052) (width 0.635) (layer F.Cu) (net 12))
 (segment (start 198.848 39.116) (end 198.912 39.052) (width 0.635) (layer F.Cu) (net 12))
 (segment (start 212.725 50.165) (end 212.725 46.985) (width 0.635) (layer F.Cu) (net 11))
 (segment (start 197.698 41.052) (end 198.912 41.052) (width 0.635) (layer F.Cu) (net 11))
 (segment (start 196.81 41.94) (end 197.698 41.052) (width 0.635) (layer F.Cu) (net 11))
 (segment (start 196.81 50.35) (end 196.81 41.94) (width 0.635) (layer F.Cu) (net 11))
 (segment (start 197.56 51.1) (end 196.81 50.35) (width 0.635) (layer F.Cu) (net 11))
 (segment (start 201.52 51.1) (end 197.56 51.1) (width 0.635) (layer F.Cu) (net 11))
 (segment (start 202.48 50.14) (end 201.52 51.1) (width 0.635) (layer F.Cu) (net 11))
 (segment (start 202.48 47.553554) (end 202.48 50.14) (width 0.635) (layer F.Cu) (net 11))
 (segment (start 203.396152 46.637402) (end 202.48 47.553554) (width 0.635) (layer F.Cu) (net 11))
 (segment (start 212.377402 46.637402) (end 203.396152 46.637402) (width 0.635) (layer F.Cu) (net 11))
 (segment (start 212.725 46.985) (end 212.377402 46.637402) (width 0.635) (layer F.Cu) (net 11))
 (segment (start 198.912 43.052) (end 201.55 43.052) (width 0.635) (layer F.Cu) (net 10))
 (segment (start 203.374 41.228) (end 203.374 34.544) (width 0.635) (layer F.Cu) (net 10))
 (segment (start 201.55 43.052) (end 203.374 41.228) (width 0.635) (layer F.Cu) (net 10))
 (segment (start 198.912 43.052) (end 197.994 43.052) (width 0.635) (layer F.Cu) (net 10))
 (segment (start 215.716 44.244) (end 220.472 44.244) (width 0.635) (layer F.Cu) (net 10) (status 20))
 (segment (start 214.11 45.85) (end 215.716 44.244) (width 0.635) (layer F.Cu) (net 10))
 (segment (start 203.07 45.85) (end 214.11 45.85) (width 0.635) (layer F.Cu) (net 10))
 (segment (start 201.676 47.244) (end 203.07 45.85) (width 0.635) (layer F.Cu) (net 10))
 (segment (start 201.676 49.784) (end 201.676 47.244) (width 0.635) (layer F.Cu) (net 10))
 (segment (start 201.168 50.292) (end 201.676 49.784) (width 0.635) (layer F.Cu) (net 10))
 (segment (start 197.866 50.292) (end 201.168 50.292) (width 0.635) (layer F.Cu) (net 10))
 (segment (start 197.612 50.038) (end 197.866 50.292) (width 0.635) (layer F.Cu) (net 10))
 (segment (start 197.612 43.434) (end 197.612 50.038) (width 0.635) (layer F.Cu) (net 10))
 (segment (start 197.994 43.052) (end 197.612 43.434) (width 0.635) (layer F.Cu) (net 10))
 (segment (start 171.276 38.1) (end 181.61 38.1) (width 0.635) (layer F.Cu) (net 2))
 (segment (start 182.658 37.052) (end 184.912 37.052) (width 0.635) (layer F.Cu) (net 2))
 (segment (start 181.61 38.1) (end 182.658 37.052) (width 0.635) (layer F.Cu) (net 2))
 (segment (start 171.276 34.798) (end 171.276 38.1) (width 0.635) (layer F.Cu) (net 2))
 (segment (start 205.994 42.244) (end 203.628 42.244) (width 0.635) (layer F.Cu) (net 9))
 (segment (start 203.628 42.244) (end 200.82 45.052) (width 0.635) (layer F.Cu) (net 9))
 (segment (start 200.82 45.052) (end 198.912 45.052) (width 0.635) (layer F.Cu) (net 9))
 (segment (start 208.534 42.244) (end 208.534 42.926) (width 0.635) (layer F.Cu) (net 8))
 (segment (start 208.534 42.926) (end 207.772 43.688) (width 0.635) (layer F.Cu) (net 8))
 (segment (start 207.772 43.688) (end 203.962 43.688) (width 0.635) (layer F.Cu) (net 8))
 (segment (start 203.962 43.688) (end 200.598 47.052) (width 0.635) (layer F.Cu) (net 8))
 (segment (start 200.598 47.052) (end 198.912 47.052) (width 0.635) (layer F.Cu) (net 8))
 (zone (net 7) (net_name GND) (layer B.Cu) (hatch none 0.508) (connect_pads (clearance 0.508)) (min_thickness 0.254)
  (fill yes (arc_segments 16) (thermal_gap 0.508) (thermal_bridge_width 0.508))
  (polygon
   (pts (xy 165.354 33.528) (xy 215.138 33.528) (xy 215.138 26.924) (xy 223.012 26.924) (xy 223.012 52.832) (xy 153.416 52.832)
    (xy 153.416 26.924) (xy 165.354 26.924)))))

